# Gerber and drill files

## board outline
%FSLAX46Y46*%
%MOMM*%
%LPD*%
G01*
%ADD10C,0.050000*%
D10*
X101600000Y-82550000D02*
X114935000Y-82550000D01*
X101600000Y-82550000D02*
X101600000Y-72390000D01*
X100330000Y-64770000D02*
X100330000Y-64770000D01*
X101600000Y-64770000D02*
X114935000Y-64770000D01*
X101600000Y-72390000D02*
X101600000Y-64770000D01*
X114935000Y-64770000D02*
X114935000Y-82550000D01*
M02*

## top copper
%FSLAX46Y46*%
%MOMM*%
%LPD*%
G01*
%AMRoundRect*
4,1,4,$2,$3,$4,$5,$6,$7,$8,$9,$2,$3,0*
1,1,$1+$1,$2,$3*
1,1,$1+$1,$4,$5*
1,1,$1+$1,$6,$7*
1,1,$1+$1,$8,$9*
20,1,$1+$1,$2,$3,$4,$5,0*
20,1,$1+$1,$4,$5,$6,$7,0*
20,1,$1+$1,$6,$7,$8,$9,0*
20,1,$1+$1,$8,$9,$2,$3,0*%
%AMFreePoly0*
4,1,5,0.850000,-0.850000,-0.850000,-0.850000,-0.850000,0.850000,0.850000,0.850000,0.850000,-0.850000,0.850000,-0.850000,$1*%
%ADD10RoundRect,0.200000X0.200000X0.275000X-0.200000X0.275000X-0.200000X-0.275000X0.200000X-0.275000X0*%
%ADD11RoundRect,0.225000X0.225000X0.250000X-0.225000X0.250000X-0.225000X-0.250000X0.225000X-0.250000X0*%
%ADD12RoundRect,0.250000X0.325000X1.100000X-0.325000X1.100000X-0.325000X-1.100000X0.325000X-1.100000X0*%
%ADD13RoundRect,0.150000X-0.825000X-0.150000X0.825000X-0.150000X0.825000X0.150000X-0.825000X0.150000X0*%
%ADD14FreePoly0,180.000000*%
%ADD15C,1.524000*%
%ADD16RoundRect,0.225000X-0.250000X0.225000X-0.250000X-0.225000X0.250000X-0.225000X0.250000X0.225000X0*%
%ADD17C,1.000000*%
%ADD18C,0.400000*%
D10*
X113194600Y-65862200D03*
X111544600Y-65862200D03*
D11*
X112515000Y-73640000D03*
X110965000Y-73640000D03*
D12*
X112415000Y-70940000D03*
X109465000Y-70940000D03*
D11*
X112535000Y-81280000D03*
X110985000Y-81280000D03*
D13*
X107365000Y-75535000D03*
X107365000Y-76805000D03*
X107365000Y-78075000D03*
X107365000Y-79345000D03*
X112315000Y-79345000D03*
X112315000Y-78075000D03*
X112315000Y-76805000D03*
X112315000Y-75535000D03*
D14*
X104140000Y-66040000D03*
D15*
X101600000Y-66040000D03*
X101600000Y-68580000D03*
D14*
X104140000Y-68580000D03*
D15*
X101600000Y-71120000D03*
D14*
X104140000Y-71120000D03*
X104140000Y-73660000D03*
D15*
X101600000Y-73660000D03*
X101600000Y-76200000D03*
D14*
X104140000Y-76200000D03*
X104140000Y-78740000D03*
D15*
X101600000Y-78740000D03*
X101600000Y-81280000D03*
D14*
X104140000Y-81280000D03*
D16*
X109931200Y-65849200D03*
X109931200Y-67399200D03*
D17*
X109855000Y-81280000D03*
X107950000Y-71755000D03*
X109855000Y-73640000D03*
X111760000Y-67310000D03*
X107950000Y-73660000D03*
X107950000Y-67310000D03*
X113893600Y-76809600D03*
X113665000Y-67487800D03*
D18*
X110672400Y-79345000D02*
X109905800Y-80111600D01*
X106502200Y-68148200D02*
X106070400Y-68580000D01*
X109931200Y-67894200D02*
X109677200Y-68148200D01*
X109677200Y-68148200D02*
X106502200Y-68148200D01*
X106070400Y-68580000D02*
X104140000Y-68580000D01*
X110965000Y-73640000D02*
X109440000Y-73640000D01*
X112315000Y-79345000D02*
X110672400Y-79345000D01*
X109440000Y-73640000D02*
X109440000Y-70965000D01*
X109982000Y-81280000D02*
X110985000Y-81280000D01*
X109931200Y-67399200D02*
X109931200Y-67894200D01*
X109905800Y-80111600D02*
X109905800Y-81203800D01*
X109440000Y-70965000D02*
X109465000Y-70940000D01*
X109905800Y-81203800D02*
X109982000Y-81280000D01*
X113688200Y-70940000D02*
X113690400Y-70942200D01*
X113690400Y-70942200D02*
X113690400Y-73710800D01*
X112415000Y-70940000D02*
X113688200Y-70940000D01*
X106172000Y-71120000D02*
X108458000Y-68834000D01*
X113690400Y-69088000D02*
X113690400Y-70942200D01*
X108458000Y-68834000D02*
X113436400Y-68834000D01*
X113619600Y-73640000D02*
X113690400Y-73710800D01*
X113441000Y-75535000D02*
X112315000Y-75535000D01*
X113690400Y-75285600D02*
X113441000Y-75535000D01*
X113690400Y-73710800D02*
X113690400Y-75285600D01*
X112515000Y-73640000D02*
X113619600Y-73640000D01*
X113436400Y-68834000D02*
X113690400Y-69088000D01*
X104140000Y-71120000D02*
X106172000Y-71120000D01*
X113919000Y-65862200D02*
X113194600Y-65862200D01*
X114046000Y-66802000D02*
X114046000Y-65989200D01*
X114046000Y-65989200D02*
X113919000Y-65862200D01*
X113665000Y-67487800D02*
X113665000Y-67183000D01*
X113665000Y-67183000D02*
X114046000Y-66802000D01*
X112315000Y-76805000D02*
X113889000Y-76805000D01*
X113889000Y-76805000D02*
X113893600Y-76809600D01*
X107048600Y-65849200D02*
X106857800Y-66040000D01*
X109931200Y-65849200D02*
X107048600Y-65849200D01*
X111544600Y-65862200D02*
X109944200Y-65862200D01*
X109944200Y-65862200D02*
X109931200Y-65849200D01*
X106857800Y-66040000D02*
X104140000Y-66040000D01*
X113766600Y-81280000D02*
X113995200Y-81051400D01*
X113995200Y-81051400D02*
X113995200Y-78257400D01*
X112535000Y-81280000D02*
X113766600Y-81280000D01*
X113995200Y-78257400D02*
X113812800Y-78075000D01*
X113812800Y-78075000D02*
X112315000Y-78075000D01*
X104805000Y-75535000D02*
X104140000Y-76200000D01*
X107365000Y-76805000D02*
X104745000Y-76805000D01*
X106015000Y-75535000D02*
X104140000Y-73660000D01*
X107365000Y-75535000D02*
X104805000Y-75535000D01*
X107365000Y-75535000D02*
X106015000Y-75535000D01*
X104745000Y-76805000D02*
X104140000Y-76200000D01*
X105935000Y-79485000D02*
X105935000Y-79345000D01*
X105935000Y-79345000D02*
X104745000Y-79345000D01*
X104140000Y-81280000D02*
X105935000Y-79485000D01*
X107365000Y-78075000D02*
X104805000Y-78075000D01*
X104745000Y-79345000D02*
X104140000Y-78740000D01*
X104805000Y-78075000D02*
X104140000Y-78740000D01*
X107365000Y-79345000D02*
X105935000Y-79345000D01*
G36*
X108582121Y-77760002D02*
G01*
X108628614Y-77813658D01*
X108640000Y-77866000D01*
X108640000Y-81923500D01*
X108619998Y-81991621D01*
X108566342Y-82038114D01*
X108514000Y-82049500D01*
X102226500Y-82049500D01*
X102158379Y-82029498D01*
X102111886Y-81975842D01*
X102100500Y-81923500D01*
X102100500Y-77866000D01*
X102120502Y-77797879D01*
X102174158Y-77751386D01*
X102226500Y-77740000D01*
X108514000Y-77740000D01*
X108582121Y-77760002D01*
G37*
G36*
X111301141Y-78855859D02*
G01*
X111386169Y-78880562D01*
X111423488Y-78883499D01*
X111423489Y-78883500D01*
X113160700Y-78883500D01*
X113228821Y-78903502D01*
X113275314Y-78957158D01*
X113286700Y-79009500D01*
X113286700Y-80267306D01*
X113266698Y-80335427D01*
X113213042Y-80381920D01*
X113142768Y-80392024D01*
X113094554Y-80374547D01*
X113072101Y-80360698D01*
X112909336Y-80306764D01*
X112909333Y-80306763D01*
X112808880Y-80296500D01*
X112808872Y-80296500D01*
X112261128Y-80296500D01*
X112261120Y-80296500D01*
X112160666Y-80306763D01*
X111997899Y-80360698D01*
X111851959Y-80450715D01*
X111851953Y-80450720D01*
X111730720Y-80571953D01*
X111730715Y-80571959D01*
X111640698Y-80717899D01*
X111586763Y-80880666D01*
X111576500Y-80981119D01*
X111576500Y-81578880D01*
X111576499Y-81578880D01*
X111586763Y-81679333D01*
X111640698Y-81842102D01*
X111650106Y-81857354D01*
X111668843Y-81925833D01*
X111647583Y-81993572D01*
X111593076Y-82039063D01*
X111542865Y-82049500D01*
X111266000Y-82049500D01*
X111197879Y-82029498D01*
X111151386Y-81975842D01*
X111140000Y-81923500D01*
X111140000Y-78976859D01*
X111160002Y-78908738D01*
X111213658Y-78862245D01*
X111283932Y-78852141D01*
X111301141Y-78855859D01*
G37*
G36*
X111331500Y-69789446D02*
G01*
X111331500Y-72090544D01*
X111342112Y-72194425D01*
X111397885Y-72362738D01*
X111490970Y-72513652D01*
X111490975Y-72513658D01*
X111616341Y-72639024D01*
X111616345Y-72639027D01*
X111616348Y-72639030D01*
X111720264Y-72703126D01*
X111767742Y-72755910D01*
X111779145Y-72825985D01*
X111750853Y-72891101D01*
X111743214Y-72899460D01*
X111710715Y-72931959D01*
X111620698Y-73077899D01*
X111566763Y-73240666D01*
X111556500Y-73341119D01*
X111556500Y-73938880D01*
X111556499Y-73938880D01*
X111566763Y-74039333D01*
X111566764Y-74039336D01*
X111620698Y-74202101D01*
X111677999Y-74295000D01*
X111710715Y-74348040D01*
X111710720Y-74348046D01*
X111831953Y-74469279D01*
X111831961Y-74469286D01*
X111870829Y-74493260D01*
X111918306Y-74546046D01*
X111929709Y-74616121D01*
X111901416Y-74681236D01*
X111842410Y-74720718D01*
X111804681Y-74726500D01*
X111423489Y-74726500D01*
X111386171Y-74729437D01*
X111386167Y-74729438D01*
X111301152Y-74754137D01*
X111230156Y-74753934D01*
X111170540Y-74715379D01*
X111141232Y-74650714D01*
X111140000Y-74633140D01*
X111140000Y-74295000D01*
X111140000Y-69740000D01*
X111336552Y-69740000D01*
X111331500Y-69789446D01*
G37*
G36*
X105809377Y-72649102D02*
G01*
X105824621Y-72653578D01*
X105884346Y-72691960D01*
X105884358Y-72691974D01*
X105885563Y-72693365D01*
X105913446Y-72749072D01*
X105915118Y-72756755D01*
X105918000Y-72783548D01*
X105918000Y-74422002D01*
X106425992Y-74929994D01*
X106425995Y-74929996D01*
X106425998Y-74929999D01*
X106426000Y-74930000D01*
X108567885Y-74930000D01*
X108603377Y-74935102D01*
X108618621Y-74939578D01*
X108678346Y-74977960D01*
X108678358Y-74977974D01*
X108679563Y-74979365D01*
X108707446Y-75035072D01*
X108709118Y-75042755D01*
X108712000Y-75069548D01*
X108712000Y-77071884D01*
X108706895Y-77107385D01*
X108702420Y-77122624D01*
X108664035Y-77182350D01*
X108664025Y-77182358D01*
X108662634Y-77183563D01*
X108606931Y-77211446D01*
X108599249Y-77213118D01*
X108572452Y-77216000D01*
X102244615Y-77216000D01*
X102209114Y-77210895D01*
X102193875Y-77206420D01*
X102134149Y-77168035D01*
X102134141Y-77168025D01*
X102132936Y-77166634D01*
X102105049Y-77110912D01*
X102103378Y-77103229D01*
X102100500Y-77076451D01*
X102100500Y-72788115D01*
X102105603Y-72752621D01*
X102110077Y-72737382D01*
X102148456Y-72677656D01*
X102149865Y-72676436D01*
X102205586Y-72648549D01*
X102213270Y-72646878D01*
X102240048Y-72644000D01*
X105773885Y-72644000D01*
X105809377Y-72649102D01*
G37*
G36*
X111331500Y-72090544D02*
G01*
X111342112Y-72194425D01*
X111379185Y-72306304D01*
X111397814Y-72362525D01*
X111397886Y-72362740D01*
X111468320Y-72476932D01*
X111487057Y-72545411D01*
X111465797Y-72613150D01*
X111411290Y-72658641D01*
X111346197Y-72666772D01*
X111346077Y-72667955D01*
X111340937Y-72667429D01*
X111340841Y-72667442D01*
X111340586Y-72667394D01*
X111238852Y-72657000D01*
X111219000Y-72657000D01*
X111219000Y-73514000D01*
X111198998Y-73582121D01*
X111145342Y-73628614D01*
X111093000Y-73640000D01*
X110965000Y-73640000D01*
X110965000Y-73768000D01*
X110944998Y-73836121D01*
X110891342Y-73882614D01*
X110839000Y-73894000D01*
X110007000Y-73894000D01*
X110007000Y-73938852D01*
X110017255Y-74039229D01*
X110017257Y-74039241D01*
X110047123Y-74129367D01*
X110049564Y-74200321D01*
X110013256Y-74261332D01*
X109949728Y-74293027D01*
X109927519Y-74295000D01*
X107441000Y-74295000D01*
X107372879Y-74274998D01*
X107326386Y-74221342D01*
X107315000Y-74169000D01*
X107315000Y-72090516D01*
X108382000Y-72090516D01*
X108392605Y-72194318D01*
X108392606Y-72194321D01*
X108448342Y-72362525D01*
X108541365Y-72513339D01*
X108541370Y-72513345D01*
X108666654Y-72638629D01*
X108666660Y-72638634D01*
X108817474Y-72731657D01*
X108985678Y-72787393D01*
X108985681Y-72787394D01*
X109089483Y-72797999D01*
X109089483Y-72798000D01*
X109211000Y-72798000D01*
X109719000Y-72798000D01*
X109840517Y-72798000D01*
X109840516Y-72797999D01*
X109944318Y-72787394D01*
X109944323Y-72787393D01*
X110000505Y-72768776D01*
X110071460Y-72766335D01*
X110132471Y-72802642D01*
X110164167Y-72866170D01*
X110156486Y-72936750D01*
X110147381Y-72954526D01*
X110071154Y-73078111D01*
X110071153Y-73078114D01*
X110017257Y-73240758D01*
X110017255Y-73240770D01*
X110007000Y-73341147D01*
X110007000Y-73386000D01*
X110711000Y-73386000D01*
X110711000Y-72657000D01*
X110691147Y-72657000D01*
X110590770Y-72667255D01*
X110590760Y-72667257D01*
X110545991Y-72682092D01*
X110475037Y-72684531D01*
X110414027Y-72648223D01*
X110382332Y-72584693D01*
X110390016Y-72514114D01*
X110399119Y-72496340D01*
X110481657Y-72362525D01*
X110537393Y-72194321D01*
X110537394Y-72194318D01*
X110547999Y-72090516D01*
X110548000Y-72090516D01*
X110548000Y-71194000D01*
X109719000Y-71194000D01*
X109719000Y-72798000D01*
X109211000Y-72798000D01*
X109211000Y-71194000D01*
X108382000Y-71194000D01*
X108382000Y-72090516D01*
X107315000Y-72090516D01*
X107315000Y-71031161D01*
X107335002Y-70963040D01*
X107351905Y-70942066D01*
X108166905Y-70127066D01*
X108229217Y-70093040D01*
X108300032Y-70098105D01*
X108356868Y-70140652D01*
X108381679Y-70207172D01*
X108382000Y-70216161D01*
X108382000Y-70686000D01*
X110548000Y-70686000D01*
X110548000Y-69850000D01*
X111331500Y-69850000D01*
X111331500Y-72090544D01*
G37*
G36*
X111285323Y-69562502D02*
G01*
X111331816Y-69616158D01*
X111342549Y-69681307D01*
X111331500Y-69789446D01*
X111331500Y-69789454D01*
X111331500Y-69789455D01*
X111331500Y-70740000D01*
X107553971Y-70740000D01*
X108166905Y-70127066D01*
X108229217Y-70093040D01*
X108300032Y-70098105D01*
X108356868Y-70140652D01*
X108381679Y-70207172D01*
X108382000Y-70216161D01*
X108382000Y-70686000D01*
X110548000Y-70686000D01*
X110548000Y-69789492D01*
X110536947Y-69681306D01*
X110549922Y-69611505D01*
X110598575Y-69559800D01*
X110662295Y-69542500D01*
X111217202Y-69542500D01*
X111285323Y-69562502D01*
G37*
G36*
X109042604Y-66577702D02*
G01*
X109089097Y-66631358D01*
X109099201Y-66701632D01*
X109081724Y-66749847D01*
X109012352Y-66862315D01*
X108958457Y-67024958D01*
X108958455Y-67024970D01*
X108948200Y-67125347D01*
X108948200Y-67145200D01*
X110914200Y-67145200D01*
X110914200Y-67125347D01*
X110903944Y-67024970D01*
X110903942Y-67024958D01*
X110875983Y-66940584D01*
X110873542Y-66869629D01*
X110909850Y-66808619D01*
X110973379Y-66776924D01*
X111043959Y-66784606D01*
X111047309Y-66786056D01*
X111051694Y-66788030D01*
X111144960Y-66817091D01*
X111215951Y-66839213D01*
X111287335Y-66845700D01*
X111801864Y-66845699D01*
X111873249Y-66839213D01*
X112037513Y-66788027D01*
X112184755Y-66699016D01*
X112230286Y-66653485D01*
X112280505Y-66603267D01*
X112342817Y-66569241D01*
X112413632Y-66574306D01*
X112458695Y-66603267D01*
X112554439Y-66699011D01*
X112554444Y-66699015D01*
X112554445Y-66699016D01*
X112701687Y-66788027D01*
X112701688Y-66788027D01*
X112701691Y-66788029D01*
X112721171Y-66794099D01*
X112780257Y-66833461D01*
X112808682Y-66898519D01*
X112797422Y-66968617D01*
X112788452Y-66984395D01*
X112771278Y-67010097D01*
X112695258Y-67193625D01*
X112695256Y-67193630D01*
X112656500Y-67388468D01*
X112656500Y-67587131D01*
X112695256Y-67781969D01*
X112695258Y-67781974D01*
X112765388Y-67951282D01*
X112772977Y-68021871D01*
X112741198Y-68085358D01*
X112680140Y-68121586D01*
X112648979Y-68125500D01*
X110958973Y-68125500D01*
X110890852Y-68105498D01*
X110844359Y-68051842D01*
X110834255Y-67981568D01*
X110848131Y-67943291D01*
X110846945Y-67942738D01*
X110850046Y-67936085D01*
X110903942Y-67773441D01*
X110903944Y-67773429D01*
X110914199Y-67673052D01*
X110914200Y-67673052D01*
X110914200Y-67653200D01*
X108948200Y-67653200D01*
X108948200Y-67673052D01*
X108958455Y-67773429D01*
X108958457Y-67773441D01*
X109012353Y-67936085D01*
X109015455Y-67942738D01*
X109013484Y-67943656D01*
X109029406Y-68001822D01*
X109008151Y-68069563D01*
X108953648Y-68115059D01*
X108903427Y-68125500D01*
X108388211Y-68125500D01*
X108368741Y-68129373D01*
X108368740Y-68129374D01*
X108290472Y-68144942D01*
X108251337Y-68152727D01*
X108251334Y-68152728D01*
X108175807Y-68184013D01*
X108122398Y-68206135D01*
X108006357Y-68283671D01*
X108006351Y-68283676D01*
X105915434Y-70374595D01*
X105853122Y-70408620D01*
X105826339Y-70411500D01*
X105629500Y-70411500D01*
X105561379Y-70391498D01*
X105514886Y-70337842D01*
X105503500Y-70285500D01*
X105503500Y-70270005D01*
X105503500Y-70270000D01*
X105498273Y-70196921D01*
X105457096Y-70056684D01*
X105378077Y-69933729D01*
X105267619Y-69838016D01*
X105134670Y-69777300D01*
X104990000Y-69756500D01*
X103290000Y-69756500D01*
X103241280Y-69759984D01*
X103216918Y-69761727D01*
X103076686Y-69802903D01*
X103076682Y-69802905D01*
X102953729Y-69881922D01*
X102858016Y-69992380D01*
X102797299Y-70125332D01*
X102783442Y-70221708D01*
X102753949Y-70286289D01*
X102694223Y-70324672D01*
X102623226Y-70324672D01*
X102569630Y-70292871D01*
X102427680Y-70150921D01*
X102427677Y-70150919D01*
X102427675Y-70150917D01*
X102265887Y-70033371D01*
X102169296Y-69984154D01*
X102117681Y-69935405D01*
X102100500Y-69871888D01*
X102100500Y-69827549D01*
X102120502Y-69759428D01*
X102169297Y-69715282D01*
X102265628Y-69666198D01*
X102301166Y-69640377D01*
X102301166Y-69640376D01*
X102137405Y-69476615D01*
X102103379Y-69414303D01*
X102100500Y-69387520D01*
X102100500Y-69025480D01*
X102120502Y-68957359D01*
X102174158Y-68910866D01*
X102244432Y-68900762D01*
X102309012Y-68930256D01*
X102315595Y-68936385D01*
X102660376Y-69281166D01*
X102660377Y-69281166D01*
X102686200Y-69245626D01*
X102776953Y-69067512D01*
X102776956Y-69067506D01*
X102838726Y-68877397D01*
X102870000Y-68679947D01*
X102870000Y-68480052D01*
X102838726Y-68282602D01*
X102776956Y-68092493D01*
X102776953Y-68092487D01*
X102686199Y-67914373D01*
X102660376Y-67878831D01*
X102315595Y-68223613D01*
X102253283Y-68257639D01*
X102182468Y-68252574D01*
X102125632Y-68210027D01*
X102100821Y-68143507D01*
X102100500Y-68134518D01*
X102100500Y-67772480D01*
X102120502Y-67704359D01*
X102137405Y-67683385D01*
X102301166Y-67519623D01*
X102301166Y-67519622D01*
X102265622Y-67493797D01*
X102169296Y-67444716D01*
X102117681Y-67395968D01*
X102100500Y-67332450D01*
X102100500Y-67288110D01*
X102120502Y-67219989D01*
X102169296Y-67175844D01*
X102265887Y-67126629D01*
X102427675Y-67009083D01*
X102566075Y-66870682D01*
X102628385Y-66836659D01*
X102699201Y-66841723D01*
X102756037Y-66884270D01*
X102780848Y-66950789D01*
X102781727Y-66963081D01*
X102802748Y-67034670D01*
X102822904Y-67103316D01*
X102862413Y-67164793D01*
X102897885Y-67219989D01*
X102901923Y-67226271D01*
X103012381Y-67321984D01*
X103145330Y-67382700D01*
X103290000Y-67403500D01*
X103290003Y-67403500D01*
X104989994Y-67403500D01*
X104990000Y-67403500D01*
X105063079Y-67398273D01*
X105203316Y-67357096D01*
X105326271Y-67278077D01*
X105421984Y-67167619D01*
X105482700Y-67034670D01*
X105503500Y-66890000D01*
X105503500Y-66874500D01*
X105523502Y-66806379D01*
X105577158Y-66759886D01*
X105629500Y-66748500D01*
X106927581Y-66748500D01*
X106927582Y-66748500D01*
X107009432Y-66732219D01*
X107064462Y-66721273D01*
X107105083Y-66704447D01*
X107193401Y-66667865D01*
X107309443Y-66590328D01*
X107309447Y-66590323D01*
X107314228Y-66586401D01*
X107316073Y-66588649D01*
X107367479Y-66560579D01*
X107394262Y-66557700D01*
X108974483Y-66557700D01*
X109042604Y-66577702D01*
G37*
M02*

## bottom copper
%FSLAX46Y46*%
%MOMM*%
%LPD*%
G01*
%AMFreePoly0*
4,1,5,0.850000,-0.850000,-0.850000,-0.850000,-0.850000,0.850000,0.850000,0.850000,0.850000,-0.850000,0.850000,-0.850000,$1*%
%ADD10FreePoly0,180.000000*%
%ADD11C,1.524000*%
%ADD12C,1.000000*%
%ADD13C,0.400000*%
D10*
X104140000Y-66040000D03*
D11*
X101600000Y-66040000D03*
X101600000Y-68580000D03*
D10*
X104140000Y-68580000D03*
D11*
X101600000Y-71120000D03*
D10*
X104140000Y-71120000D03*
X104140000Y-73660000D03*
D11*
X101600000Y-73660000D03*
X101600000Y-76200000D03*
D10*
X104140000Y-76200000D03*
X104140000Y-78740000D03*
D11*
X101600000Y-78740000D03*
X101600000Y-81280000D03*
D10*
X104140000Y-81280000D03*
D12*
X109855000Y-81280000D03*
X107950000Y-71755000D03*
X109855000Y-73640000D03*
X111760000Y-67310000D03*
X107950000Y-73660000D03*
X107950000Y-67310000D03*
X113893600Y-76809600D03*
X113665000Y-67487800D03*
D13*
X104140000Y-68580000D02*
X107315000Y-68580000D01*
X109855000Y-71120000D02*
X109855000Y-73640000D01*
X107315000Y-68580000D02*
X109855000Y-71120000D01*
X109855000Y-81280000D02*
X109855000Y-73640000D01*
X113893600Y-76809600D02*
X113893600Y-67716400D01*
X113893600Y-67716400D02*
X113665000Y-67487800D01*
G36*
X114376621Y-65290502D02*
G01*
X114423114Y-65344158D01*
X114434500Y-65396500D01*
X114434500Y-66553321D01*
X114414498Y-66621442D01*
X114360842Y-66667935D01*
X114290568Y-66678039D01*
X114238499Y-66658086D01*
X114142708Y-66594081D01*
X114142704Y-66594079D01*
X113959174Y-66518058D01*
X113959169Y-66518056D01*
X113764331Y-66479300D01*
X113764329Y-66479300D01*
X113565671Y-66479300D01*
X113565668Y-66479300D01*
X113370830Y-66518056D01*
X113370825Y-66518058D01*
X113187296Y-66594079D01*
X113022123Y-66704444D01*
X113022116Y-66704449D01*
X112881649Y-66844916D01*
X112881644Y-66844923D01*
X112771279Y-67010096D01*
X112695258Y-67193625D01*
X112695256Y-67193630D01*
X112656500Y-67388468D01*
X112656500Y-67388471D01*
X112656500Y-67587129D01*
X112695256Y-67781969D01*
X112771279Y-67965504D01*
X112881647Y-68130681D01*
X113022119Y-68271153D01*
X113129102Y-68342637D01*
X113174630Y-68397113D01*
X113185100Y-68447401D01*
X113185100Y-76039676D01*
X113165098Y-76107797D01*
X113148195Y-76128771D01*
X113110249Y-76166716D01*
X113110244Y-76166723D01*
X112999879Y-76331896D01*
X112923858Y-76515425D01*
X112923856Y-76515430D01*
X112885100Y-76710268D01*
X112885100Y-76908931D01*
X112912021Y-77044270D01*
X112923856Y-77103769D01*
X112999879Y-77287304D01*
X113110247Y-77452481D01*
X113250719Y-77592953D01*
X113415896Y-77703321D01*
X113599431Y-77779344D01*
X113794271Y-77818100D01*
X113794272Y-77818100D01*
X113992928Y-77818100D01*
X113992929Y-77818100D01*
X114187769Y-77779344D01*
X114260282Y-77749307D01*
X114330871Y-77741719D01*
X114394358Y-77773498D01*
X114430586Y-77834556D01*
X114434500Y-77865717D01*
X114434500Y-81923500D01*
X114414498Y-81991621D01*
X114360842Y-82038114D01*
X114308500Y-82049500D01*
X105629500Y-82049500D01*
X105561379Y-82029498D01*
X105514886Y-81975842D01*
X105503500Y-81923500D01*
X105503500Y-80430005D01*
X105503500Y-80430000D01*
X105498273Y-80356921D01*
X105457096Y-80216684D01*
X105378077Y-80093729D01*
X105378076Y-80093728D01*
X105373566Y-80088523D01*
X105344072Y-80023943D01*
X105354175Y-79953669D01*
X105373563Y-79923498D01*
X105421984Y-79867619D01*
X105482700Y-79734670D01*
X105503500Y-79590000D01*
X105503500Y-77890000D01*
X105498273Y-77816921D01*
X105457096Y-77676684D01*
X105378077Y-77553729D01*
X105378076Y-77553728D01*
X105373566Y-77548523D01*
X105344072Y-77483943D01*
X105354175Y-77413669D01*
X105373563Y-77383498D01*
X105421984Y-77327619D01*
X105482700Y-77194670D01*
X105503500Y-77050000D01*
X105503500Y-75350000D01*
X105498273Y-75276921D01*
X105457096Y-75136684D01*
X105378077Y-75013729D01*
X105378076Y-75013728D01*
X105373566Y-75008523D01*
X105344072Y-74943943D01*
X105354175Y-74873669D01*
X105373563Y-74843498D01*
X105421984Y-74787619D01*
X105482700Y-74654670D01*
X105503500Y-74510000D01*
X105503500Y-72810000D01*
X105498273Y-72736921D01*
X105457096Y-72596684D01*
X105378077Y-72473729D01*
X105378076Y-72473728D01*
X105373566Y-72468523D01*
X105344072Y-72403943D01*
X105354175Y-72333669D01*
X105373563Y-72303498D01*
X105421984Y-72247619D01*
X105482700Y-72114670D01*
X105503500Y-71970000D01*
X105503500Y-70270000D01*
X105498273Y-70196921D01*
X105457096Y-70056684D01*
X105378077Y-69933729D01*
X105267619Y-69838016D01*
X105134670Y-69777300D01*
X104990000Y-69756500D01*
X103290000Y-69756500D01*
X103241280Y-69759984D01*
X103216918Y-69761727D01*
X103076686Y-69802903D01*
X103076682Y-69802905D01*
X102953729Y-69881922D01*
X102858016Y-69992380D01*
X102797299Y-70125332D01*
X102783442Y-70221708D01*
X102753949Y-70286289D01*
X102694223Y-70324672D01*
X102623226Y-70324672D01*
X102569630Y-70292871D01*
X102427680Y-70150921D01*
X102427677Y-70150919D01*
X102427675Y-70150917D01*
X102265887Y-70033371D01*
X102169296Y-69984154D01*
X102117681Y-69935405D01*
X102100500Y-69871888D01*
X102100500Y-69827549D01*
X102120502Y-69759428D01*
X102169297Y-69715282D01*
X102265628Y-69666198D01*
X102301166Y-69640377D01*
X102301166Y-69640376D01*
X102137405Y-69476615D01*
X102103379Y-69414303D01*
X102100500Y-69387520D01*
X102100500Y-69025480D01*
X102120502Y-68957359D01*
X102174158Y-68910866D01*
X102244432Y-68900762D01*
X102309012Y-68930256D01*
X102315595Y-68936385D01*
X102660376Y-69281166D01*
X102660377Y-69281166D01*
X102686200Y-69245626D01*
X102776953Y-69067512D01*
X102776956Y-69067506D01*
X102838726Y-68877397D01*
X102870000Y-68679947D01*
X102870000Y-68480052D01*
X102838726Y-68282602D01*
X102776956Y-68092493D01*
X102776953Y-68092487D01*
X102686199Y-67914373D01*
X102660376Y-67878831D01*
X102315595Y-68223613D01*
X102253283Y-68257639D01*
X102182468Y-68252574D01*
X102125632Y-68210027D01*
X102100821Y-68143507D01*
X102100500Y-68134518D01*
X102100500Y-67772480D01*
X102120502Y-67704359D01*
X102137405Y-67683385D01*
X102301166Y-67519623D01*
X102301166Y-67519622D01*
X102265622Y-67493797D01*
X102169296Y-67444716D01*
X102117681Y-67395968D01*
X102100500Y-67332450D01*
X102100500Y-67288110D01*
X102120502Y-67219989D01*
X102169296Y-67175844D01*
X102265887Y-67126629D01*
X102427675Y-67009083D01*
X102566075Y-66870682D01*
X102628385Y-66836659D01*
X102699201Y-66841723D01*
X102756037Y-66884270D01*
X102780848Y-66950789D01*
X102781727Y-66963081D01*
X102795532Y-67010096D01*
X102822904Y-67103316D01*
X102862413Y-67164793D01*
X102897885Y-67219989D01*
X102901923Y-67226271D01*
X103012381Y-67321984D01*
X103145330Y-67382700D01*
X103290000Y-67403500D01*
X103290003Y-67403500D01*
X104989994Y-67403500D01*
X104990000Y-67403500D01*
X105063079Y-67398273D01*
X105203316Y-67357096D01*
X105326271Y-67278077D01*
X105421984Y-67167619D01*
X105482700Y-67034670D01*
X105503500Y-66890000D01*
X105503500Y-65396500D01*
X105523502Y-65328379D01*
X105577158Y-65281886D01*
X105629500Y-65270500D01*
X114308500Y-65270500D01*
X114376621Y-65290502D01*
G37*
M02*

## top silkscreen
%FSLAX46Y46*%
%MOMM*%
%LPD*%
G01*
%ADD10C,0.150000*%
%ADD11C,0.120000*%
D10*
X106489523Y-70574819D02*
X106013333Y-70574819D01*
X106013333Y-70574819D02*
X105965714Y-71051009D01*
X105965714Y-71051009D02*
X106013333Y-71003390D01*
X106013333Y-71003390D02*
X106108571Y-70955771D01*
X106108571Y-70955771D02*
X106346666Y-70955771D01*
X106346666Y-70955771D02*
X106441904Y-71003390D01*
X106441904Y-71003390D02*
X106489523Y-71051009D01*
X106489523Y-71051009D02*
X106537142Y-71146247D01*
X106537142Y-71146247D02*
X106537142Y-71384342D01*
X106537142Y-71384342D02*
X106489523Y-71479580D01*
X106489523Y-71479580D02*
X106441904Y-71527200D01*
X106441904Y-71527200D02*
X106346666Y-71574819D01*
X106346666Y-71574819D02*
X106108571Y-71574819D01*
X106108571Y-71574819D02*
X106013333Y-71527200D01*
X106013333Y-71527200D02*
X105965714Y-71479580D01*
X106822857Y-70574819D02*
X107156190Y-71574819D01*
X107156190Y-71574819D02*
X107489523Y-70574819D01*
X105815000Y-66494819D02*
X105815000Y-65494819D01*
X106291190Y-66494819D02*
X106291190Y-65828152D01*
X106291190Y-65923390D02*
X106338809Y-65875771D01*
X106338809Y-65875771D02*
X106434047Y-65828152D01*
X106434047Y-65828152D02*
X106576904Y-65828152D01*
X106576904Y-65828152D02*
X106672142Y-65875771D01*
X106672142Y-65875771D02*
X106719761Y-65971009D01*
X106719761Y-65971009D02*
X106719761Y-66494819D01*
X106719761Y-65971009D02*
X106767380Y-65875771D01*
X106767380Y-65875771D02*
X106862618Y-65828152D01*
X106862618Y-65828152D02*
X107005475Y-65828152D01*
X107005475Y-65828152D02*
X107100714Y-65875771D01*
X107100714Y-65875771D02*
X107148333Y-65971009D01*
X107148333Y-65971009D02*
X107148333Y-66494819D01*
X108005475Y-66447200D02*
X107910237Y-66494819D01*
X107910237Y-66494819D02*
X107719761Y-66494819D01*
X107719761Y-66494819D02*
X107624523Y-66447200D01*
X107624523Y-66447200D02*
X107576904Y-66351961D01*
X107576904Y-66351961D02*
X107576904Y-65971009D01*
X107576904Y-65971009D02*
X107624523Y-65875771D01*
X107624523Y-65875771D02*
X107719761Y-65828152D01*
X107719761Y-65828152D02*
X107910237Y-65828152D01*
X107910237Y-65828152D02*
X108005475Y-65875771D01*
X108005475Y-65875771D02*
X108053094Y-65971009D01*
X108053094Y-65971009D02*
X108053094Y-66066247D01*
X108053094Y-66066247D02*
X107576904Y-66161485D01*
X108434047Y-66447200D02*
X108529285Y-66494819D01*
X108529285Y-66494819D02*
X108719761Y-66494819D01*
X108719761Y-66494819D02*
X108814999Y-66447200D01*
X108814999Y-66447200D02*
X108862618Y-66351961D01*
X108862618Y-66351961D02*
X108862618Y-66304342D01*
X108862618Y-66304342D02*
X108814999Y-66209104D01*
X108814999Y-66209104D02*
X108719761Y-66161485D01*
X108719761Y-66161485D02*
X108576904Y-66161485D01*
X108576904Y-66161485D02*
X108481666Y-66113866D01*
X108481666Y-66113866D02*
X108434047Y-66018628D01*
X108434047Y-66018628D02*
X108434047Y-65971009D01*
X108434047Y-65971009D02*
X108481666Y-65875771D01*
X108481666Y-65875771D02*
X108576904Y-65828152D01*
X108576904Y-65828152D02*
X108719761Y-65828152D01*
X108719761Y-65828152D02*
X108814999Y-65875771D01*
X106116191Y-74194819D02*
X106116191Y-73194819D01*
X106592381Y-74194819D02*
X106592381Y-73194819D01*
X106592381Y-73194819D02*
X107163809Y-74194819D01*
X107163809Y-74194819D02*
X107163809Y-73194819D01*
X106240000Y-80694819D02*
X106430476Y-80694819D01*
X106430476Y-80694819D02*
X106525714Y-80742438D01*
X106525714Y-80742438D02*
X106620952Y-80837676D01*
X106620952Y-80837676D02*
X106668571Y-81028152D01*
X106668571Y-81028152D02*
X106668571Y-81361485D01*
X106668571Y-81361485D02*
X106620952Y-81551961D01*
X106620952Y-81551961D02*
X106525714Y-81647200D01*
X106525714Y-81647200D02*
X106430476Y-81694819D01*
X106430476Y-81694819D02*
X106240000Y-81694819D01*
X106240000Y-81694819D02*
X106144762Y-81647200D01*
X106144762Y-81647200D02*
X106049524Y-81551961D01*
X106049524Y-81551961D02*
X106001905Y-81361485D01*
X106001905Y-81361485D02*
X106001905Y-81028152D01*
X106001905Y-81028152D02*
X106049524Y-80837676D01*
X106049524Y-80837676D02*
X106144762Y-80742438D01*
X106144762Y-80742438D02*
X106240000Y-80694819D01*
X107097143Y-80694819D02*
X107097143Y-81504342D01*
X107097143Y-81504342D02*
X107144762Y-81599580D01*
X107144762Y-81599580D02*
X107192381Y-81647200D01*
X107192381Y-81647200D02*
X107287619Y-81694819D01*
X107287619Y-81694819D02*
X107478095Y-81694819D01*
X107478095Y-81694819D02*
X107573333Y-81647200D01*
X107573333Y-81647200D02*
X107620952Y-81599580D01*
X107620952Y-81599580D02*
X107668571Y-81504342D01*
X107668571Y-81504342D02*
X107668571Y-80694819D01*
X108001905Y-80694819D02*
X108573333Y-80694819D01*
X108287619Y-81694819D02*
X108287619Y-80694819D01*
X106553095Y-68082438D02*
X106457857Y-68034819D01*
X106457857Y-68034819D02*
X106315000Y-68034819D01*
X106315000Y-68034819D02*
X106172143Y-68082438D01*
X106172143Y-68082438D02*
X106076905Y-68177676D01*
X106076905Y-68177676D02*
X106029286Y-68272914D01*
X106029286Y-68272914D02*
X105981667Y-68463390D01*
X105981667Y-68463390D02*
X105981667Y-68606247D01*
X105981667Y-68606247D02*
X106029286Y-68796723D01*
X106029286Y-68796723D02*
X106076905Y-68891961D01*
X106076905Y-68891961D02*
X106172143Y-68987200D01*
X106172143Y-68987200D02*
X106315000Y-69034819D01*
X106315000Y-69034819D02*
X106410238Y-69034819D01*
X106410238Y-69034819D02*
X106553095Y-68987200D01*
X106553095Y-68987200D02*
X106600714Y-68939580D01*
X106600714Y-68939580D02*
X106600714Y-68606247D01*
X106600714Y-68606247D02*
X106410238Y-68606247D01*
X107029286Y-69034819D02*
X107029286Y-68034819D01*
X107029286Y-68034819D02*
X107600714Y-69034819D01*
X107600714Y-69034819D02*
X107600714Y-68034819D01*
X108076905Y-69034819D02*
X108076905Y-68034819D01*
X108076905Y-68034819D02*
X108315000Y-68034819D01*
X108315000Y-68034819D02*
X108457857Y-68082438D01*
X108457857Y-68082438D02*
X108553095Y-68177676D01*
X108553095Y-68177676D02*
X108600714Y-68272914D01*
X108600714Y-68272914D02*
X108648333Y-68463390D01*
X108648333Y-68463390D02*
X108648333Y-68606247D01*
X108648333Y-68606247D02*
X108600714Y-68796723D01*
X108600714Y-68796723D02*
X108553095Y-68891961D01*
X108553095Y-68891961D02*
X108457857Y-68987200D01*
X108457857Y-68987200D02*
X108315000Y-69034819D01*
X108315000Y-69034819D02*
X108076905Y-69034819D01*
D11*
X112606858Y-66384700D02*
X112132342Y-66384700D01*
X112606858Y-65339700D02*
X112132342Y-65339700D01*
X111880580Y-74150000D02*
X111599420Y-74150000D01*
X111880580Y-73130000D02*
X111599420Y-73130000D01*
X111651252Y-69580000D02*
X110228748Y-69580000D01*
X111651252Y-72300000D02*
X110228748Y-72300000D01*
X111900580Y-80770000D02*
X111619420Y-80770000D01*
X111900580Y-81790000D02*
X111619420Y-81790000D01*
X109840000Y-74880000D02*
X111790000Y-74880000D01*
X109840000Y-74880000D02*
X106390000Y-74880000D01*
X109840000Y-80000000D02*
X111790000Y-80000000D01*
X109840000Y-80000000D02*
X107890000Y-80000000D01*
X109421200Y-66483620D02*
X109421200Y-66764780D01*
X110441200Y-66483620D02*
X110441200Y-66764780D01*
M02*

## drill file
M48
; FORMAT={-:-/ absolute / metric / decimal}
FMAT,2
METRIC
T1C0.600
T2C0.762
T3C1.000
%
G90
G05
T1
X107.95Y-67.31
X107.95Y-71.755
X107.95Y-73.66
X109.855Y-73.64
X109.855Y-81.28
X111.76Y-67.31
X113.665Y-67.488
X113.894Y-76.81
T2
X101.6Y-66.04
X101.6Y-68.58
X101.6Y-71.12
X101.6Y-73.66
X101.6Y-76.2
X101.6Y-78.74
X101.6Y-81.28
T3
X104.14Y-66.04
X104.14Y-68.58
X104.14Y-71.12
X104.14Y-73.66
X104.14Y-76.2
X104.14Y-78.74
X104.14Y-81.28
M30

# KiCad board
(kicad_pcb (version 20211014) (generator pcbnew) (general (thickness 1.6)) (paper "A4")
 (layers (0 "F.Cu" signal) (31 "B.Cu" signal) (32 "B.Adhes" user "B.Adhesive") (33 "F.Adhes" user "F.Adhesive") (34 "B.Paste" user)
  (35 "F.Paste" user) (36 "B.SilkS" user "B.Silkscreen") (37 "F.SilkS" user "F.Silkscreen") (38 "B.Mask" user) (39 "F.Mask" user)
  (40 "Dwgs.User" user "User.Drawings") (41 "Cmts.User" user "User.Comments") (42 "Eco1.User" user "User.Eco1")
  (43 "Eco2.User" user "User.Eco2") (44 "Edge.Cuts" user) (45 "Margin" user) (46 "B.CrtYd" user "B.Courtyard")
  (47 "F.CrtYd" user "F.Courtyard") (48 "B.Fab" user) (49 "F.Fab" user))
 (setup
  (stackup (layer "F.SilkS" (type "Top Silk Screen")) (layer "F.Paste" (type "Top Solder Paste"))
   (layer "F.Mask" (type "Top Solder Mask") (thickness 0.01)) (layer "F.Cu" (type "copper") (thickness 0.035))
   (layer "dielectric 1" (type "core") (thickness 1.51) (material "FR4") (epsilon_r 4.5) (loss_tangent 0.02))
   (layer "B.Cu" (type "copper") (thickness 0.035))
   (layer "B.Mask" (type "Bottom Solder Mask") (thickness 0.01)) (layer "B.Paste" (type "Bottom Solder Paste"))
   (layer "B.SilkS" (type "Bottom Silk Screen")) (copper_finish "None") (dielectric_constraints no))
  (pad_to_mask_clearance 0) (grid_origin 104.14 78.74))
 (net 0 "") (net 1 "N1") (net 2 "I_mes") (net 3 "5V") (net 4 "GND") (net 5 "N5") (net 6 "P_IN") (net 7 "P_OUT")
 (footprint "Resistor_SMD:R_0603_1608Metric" (layer "F.Cu") (at 112.3696 65.8622 180)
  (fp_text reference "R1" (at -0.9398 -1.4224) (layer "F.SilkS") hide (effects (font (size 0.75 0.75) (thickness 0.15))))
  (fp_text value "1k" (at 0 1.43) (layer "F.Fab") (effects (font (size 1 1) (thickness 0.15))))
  (fp_line (start -0.237258 -0.5225) (end 0.237258 -0.5225) (layer "F.SilkS") (width 0.12))
  (fp_line (start -0.237258 0.5225) (end 0.237258 0.5225) (layer "F.SilkS") (width 0.12))
  (pad "1" smd roundrect (at -0.825 0 180) (size 0.8 0.95) (layers "F.Cu" "F.Paste" "F.Mask") (roundrect_rratio 0.25) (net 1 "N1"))
  (pad "2" smd roundrect (at 0.825 0 180) (size 0.8 0.95) (layers "F.Cu" "F.Paste" "F.Mask") (roundrect_rratio 0.25) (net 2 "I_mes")))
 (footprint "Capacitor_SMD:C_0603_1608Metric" (layer "F.Cu") (at 111.74 73.64 180)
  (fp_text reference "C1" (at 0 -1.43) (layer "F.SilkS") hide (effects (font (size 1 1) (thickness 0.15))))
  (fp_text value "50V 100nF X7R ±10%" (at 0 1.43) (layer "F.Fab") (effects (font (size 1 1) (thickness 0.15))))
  (fp_line (start -0.14058 -0.51) (end 0.14058 -0.51) (layer "F.SilkS") (width 0.12))
  (fp_line (start -0.14058 0.51) (end 0.14058 0.51) (layer "F.SilkS") (width 0.12))
  (pad "1" smd roundrect (at -0.775 0 180) (size 0.9 0.95) (layers "F.Cu" "F.Paste" "F.Mask") (roundrect_rratio 0.25) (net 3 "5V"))
  (pad "2" smd roundrect (at 0.775 0 180) (size 0.9 0.95) (layers "F.Cu" "F.Paste" "F.Mask") (roundrect_rratio 0.25) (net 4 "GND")))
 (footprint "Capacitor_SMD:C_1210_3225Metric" (layer "F.Cu") (at 110.94 70.94 180)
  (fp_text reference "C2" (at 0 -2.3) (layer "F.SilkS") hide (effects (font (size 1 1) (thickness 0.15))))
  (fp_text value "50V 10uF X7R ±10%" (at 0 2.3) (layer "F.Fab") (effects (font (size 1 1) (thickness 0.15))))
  (fp_line (start -0.711252 1.36) (end 0.711252 1.36) (layer "F.SilkS") (width 0.12))
  (fp_line (start -0.711252 -1.36) (end 0.711252 -1.36) (layer "F.SilkS") (width 0.12))
  (pad "1" smd roundrect (at -1.475 0 180) (size 1.15 2.7) (layers "F.Cu" "F.Paste" "F.Mask") (roundrect_rratio 0.2173913043) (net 3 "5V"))
  (pad "2" smd roundrect (at 1.475 0 180) (size 1.15 2.7) (layers "F.Cu" "F.Paste" "F.Mask") (roundrect_rratio 0.2173913043) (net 4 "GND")))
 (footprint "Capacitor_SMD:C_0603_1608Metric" (layer "F.Cu") (at 111.76 81.28 180)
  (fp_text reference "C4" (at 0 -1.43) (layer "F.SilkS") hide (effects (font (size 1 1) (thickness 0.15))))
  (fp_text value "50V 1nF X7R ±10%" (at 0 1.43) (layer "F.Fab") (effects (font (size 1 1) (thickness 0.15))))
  (fp_line (start -0.14058 0.51) (end 0.14058 0.51) (layer "F.SilkS") (width 0.12))
  (fp_line (start -0.14058 -0.51) (end 0.14058 -0.51) (layer "F.SilkS") (width 0.12))
  (pad "1" smd roundrect (at -0.775 0 180) (size 0.9 0.95) (layers "F.Cu" "F.Paste" "F.Mask") (roundrect_rratio 0.25) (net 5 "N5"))
  (pad "2" smd roundrect (at 0.775 0 180) (size 0.9 0.95) (layers "F.Cu" "F.Paste" "F.Mask") (roundrect_rratio 0.25) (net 4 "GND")))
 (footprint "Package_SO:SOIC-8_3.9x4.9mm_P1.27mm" (layer "F.Cu") (at 109.84 77.44)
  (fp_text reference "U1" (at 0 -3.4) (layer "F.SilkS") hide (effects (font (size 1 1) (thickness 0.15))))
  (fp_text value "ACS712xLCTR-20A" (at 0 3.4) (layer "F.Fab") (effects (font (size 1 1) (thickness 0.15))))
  (fp_line (start 0 -2.56) (end 1.95 -2.56) (layer "F.SilkS") (width 0.12))
  (fp_line (start 0 -2.56) (end -3.45 -2.56) (layer "F.SilkS") (width 0.12))
  (fp_line (start 0 2.56) (end 1.95 2.56) (layer "F.SilkS") (width 0.12))
  (fp_line (start 0 2.56) (end -1.95 2.56) (layer "F.SilkS") (width 0.12))
  (pad "1" smd roundrect (at -2.475 -1.905) (size 1.95 0.6) (layers "F.Cu" "F.Paste" "F.Mask") (roundrect_rratio 0.25) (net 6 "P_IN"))
  (pad "2" smd roundrect (at -2.475 -0.635) (size 1.95 0.6) (layers "F.Cu" "F.Paste" "F.Mask") (roundrect_rratio 0.25) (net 6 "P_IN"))
  (pad "3" smd roundrect (at -2.475 0.635) (size 1.95 0.6) (layers "F.Cu" "F.Paste" "F.Mask") (roundrect_rratio 0.25) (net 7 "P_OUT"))
  (pad "4" smd roundrect (at -2.475 1.905) (size 1.95 0.6) (layers "F.Cu" "F.Paste" "F.Mask") (roundrect_rratio 0.25) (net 7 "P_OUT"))
  (pad "5" smd roundrect (at 2.475 1.905) (size 1.95 0.6) (layers "F.Cu" "F.Paste" "F.Mask") (roundrect_rratio 0.25) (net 4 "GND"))
  (pad "6" smd roundrect (at 2.475 0.635) (size 1.95 0.6) (layers "F.Cu" "F.Paste" "F.Mask") (roundrect_rratio 0.25) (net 5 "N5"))
  (pad "7" smd roundrect (at 2.475 -0.635) (size 1.95 0.6) (layers "F.Cu" "F.Paste" "F.Mask") (roundrect_rratio 0.25) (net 1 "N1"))
  (pad "8" smd roundrect (at 2.475 -1.905) (size 1.95 0.6) (layers "F.Cu" "F.Paste" "F.Mask") (roundrect_rratio 0.25) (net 3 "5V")))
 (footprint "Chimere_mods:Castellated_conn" (layer "F.Cu") (at 104.14 66.04 180)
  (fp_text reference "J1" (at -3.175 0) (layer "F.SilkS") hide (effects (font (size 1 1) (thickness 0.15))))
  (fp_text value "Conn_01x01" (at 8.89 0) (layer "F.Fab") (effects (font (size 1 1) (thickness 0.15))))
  (pad "1" thru_hole custom (at 0 0 180) (size 1.7 1.7) (drill 1) (layers *.Cu *.Mask) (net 2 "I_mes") (zone_connect 2)
   (options (clearance outline) (anchor rect)) (primitives))
  (pad "1" thru_hole circle (at 2.54 0 180) (size 1.524 1.524) (drill 0.762) (layers *.Cu *.Mask) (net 2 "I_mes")))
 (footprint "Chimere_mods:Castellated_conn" (layer "F.Cu") (at 104.14 68.58 180)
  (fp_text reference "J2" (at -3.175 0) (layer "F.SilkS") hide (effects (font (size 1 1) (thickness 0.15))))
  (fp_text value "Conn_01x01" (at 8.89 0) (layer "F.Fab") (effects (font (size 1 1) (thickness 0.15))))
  (pad "1" thru_hole circle (at 2.54 0 180) (size 1.524 1.524) (drill 0.762) (layers *.Cu *.Mask) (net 4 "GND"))
  (pad "1" thru_hole custom (at 0 0 180) (size 1.7 1.7) (drill 1) (layers *.Cu *.Mask) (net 4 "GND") (zone_connect 2)
   (options (clearance outline) (anchor rect)) (primitives)))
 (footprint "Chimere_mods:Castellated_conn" (layer "F.Cu") (at 104.14 71.12 180)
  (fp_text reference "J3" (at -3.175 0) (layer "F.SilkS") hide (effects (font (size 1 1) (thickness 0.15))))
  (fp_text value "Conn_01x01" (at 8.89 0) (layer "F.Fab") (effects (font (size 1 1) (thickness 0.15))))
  (pad "1" thru_hole circle (at 2.54 0 180) (size 1.524 1.524) (drill 0.762) (layers *.Cu *.Mask) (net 3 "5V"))
  (pad "1" thru_hole custom (at 0 0 180) (size 1.7 1.7) (drill 1) (layers *.Cu *.Mask) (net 3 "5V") (zone_connect 2)
   (options (clearance outline) (anchor rect)) (primitives)))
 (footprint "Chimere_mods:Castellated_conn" (layer "F.Cu") (at 104.14 73.66 180)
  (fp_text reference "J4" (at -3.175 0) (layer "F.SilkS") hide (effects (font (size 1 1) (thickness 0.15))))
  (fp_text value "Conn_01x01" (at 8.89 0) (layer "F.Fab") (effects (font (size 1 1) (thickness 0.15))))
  (pad "1" thru_hole custom (at 0 0 180) (size 1.7 1.7) (drill 1) (layers *.Cu *.Mask) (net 6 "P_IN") (zone_connect 2)
   (options (clearance outline) (anchor rect)) (primitives))
  (pad "1" thru_hole circle (at 2.54 0 180) (size 1.524 1.524) (drill 0.762) (layers *.Cu *.Mask) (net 6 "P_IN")))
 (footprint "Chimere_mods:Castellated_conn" (layer "F.Cu") (at 104.14 76.2 180)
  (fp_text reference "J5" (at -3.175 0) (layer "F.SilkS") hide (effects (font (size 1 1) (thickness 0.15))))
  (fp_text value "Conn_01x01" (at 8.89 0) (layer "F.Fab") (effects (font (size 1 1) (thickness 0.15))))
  (pad "1" thru_hole circle (at 2.54 0 180) (size 1.524 1.524) (drill 0.762) (layers *.Cu *.Mask) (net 6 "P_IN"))
  (pad "1" thru_hole custom (at 0 0 180) (size 1.7 1.7) (drill 1) (layers *.Cu *.Mask) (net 6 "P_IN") (zone_connect 2)
   (options (clearance outline) (anchor rect)) (primitives)))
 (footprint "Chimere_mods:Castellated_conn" (layer "F.Cu") (at 104.14 78.74 180)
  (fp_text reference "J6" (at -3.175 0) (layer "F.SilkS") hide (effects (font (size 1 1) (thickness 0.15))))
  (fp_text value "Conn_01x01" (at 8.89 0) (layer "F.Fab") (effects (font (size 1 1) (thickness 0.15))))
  (pad "1" thru_hole custom (at 0 0 180) (size 1.7 1.7) (drill 1) (layers *.Cu *.Mask) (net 7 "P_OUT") (zone_connect 2)
   (options (clearance outline) (anchor rect)) (primitives))
  (pad "1" thru_hole circle (at 2.54 0 180) (size 1.524 1.524) (drill 0.762) (layers *.Cu *.Mask) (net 7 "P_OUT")))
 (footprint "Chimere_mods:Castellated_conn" (layer "F.Cu") (at 104.14 81.28 180)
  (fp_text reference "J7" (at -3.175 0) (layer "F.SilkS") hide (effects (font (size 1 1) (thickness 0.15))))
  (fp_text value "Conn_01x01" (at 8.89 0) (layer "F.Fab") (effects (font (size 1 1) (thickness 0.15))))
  (pad "1" thru_hole circle (at 2.54 0 180) (size 1.524 1.524) (drill 0.762) (layers *.Cu *.Mask) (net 7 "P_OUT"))
  (pad "1" thru_hole custom (at 0 0 180) (size 1.7 1.7) (drill 1) (layers *.Cu *.Mask) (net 7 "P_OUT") (zone_connect 2)
   (options (clearance outline) (anchor rect)) (primitives)))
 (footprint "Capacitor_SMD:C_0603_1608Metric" (layer "F.Cu") (at 109.9312 66.6242 -90)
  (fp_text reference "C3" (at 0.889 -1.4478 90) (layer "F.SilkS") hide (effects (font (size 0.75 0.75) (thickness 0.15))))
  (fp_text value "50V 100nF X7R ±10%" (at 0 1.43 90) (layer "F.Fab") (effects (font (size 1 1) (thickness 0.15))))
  (fp_line (start -0.14058 0.51) (end 0.14058 0.51) (layer "F.SilkS") (width 0.12))
  (fp_line (start -0.14058 -0.51) (end 0.14058 -0.51) (layer "F.SilkS") (width 0.12))
  (pad "1" smd roundrect (at -0.775 0 270) (size 0.9 0.95) (layers "F.Cu" "F.Paste" "F.Mask") (roundrect_rratio 0.25) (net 2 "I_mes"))
  (pad "2" smd roundrect (at 0.775 0 270) (size 0.9 0.95) (layers "F.Cu" "F.Paste" "F.Mask") (roundrect_rratio 0.25) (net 4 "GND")))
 (gr_line (start 101.6 82.55) (end 114.935 82.55) (layer "Edge.Cuts") (width 0.05))
 (gr_line (start 101.6 82.55) (end 101.6 72.39) (layer "Edge.Cuts") (width 0.05))
 (gr_line (start 100.33 64.77) (end 100.33 64.77) (layer "Edge.Cuts") (width 0.05))
 (gr_line (start 101.6 64.77) (end 114.935 64.77) (layer "Edge.Cuts") (width 0.05))
 (gr_line (start 101.6 72.39) (end 101.6 64.77) (layer "Edge.Cuts") (width 0.05))
 (gr_line (start 114.935 64.77) (end 114.935 82.55) (layer "Edge.Cuts") (width 0.05))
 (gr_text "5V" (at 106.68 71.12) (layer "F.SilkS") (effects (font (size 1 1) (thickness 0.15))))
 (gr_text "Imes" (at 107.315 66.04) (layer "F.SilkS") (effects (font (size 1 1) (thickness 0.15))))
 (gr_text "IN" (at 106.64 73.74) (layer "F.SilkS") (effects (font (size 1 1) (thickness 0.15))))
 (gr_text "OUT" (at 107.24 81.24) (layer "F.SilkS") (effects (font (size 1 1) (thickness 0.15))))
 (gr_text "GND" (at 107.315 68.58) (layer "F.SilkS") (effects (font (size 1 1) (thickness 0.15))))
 (segment (start 110.6724 79.345) (end 109.9058 80.1116) (width 0.4) (layer "F.Cu") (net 4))
 (segment (start 106.5022 68.1482) (end 106.0704 68.58) (width 0.4) (layer "F.Cu") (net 4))
 (segment (start 109.9312 67.8942) (end 109.6772 68.1482) (width 0.4) (layer "F.Cu") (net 4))
 (segment (start 109.6772 68.1482) (end 106.5022 68.1482) (width 0.4) (layer "F.Cu") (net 4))
 (segment (start 106.0704 68.58) (end 104.14 68.58) (width 0.4) (layer "F.Cu") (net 4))
 (segment (start 110.965 73.64) (end 109.44 73.64) (width 0.4) (layer "F.Cu") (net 4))
 (segment (start 112.315 79.345) (end 110.6724 79.345) (width 0.4) (layer "F.Cu") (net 4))
 (segment (start 109.44 73.64) (end 109.44 70.965) (width 0.4) (layer "F.Cu") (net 4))
 (segment (start 109.982 81.28) (end 110.985 81.28) (width 0.4) (layer "F.Cu") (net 4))
 (segment (start 109.9312 67.3992) (end 109.9312 67.8942) (width 0.4) (layer "F.Cu") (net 4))
 (segment (start 109.9058 80.1116) (end 109.9058 81.2038) (width 0.4) (layer "F.Cu") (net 4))
 (segment (start 109.44 70.965) (end 109.465 70.94) (width 0.4) (layer "F.Cu") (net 4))
 (segment (start 109.9058 81.2038) (end 109.982 81.28) (width 0.4) (layer "F.Cu") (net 4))
 (via (at 109.855 81.28) (size 1) (drill 0.6) (layers "F.Cu" "B.Cu") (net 4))
 (via (at 107.95 71.755) (size 1) (drill 0.6) (layers "F.Cu" "B.Cu") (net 4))
 (via (at 109.855 73.64) (size 1) (drill 0.6) (layers "F.Cu" "B.Cu") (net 4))
 (via (at 111.76 67.31) (size 1) (drill 0.6) (layers "F.Cu" "B.Cu") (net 4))
 (via (at 107.95 73.66) (size 1) (drill 0.6) (layers "F.Cu" "B.Cu") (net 4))
 (via (at 107.95 67.31) (size 1) (drill 0.6) (layers "F.Cu" "B.Cu") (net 4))
 (segment (start 104.14 68.58) (end 107.315 68.58) (width 0.4) (layer "B.Cu") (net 4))
 (segment (start 109.855 71.12) (end 109.855 73.64) (width 0.4) (layer "B.Cu") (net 4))
 (segment (start 107.315 68.58) (end 109.855 71.12) (width 0.4) (layer "B.Cu") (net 4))
 (segment (start 109.855 81.28) (end 109.855 73.64) (width 0.4) (layer "B.Cu") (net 4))
 (segment (start 113.6882 70.94) (end 113.6904 70.9422) (width 0.4) (layer "F.Cu") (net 3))
 (segment (start 113.6904 70.9422) (end 113.6904 73.7108) (width 0.4) (layer "F.Cu") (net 3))
 (segment (start 112.415 70.94) (end 113.6882 70.94) (width 0.4) (layer "F.Cu") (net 3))
 (segment (start 106.172 71.12) (end 108.458 68.834) (width 0.4) (layer "F.Cu") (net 3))
 (segment (start 113.6904 69.088) (end 113.6904 70.9422) (width 0.4) (layer "F.Cu") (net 3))
 (segment (start 108.458 68.834) (end 113.4364 68.834) (width 0.4) (layer "F.Cu") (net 3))
 (segment (start 113.6196 73.64) (end 113.6904 73.7108) (width 0.4) (layer "F.Cu") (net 3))
 (segment (start 113.441 75.535) (end 112.315 75.535) (width 0.4) (layer "F.Cu") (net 3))
 (segment (start 113.6904 75.2856) (end 113.441 75.535) (width 0.4) (layer "F.Cu") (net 3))
 (segment (start 113.6904 73.7108) (end 113.6904 75.2856) (width 0.4) (layer "F.Cu") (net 3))
 (segment (start 112.515 73.64) (end 113.6196 73.64) (width 0.4) (layer "F.Cu") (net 3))
 (segment (start 113.4364 68.834) (end 113.6904 69.088) (width 0.4) (layer "F.Cu") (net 3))
 (segment (start 104.14 71.12) (end 106.172 71.12) (width 0.4) (layer "F.Cu") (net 3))
 (segment (start 113.919 65.8622) (end 113.1946 65.8622) (width 0.4) (layer "F.Cu") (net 1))
 (segment (start 114.046 66.802) (end 114.046 65.9892) (width 0.4) (layer "F.Cu") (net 1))
 (segment (start 114.046 65.9892) (end 113.919 65.8622) (width 0.4) (layer "F.Cu") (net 1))
 (segment (start 113.665 67.4878) (end 113.665 67.183) (width 0.4) (layer "F.Cu") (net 1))
 (segment (start 113.665 67.183) (end 114.046 66.802) (width 0.4) (layer "F.Cu") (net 1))
 (segment (start 112.315 76.805) (end 113.889 76.805) (width 0.4) (layer "F.Cu") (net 1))
 (segment (start 113.889 76.805) (end 113.8936 76.8096) (width 0.4) (layer "F.Cu") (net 1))
 (via (at 113.8936 76.8096) (size 1) (drill 0.6) (layers "F.Cu" "B.Cu") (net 1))
 (via (at 113.665 67.4878) (size 1) (drill 0.6) (layers "F.Cu" "B.Cu") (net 1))
 (segment (start 113.8936 76.8096) (end 113.8936 67.7164) (width 0.4) (layer "B.Cu") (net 1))
 (segment (start 113.8936 67.7164) (end 113.665 67.4878) (width 0.4) (layer "B.Cu") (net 1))
 (segment (start 107.0486 65.8492) (end 106.8578 66.04) (width 0.4) (layer "F.Cu") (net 2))
 (segment (start 109.9312 65.8492) (end 107.0486 65.8492) (width 0.4) (layer "F.Cu") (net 2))
 (segment (start 111.5446 65.8622) (end 109.9442 65.8622) (width 0.4) (layer "F.Cu") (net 2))
 (segment (start 109.9442 65.8622) (end 109.9312 65.8492) (width 0.4) (layer "F.Cu") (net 2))
 (segment (start 106.8578 66.04) (end 104.14 66.04) (width 0.4) (layer "F.Cu") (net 2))
 (segment (start 113.7666 81.28) (end 113.9952 81.0514) (width 0.4) (layer "F.Cu") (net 5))
 (segment (start 113.9952 81.0514) (end 113.9952 78.2574) (width 0.4) (layer "F.Cu") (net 5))
 (segment (start 112.535 81.28) (end 113.7666 81.28) (width 0.4) (layer "F.Cu") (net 5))
 (segment (start 113.9952 78.2574) (end 113.8128 78.075) (width 0.4) (layer "F.Cu") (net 5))
 (segment (start 113.8128 78.075) (end 112.315 78.075) (width 0.4) (layer "F.Cu") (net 5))
 (segment (start 104.805 75.535) (end 104.14 76.2) (width 0.4) (layer "F.Cu") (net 6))
 (segment (start 107.365 76.805) (end 104.745 76.805) (width 0.4) (layer "F.Cu") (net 6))
 (segment (start 106.015 75.535) (end 104.14 73.66) (width 0.4) (layer "F.Cu") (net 6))
 (segment (start 107.365 75.535) (end 104.805 75.535) (width 0.4) (layer "F.Cu") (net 6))
 (segment (start 107.365 75.535) (end 106.015 75.535) (width 0.4) (layer "F.Cu") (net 6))
 (segment (start 104.745 76.805) (end 104.14 76.2) (width 0.4) (layer "F.Cu") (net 6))
 (segment (start 105.935 79.485) (end 105.935 79.345) (width 0.4) (layer "F.Cu") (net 7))
 (segment (start 105.935 79.345) (end 104.745 79.345) (width 0.4) (layer "F.Cu") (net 7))
 (segment (start 104.14 81.28) (end 105.935 79.485) (width 0.4) (layer "F.Cu") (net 7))
 (segment (start 107.365 78.075) (end 104.805 78.075) (width 0.4) (layer "F.Cu") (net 7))
 (segment (start 104.745 79.345) (end 104.14 78.74) (width 0.4) (layer "F.Cu") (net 7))
 (segment (start 104.805 78.075) (end 104.14 78.74) (width 0.4) (layer "F.Cu") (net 7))
 (segment (start 107.365 79.345) (end 105.935 79.345) (width 0.4) (layer "F.Cu") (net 7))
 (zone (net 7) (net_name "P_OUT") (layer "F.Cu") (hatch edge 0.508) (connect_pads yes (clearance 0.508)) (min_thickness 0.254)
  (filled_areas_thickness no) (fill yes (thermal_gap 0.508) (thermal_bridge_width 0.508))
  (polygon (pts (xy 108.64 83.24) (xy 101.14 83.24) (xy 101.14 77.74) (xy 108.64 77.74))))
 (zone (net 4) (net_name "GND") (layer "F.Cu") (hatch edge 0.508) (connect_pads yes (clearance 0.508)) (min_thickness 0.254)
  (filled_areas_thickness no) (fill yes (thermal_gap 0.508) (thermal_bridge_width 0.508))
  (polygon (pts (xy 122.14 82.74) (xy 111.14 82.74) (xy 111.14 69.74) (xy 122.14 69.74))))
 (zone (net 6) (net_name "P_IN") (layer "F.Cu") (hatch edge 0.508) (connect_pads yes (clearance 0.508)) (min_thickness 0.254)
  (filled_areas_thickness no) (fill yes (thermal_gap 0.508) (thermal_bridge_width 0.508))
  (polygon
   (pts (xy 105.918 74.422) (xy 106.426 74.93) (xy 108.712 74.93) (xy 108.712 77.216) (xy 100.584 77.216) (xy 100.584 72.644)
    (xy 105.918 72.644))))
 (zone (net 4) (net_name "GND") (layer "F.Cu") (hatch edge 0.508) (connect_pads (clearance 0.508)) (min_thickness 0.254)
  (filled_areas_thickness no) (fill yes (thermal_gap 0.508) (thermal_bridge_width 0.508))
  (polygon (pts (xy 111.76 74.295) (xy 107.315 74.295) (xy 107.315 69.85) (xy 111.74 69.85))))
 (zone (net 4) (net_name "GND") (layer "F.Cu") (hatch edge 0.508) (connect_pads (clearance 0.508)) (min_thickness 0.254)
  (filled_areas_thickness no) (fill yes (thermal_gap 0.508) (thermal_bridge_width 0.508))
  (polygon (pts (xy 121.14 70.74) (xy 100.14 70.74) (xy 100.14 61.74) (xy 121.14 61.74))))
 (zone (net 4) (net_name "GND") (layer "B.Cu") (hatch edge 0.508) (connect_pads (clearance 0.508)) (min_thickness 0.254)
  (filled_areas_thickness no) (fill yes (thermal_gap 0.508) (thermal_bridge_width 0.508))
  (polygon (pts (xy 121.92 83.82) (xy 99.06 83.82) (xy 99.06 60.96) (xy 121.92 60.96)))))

